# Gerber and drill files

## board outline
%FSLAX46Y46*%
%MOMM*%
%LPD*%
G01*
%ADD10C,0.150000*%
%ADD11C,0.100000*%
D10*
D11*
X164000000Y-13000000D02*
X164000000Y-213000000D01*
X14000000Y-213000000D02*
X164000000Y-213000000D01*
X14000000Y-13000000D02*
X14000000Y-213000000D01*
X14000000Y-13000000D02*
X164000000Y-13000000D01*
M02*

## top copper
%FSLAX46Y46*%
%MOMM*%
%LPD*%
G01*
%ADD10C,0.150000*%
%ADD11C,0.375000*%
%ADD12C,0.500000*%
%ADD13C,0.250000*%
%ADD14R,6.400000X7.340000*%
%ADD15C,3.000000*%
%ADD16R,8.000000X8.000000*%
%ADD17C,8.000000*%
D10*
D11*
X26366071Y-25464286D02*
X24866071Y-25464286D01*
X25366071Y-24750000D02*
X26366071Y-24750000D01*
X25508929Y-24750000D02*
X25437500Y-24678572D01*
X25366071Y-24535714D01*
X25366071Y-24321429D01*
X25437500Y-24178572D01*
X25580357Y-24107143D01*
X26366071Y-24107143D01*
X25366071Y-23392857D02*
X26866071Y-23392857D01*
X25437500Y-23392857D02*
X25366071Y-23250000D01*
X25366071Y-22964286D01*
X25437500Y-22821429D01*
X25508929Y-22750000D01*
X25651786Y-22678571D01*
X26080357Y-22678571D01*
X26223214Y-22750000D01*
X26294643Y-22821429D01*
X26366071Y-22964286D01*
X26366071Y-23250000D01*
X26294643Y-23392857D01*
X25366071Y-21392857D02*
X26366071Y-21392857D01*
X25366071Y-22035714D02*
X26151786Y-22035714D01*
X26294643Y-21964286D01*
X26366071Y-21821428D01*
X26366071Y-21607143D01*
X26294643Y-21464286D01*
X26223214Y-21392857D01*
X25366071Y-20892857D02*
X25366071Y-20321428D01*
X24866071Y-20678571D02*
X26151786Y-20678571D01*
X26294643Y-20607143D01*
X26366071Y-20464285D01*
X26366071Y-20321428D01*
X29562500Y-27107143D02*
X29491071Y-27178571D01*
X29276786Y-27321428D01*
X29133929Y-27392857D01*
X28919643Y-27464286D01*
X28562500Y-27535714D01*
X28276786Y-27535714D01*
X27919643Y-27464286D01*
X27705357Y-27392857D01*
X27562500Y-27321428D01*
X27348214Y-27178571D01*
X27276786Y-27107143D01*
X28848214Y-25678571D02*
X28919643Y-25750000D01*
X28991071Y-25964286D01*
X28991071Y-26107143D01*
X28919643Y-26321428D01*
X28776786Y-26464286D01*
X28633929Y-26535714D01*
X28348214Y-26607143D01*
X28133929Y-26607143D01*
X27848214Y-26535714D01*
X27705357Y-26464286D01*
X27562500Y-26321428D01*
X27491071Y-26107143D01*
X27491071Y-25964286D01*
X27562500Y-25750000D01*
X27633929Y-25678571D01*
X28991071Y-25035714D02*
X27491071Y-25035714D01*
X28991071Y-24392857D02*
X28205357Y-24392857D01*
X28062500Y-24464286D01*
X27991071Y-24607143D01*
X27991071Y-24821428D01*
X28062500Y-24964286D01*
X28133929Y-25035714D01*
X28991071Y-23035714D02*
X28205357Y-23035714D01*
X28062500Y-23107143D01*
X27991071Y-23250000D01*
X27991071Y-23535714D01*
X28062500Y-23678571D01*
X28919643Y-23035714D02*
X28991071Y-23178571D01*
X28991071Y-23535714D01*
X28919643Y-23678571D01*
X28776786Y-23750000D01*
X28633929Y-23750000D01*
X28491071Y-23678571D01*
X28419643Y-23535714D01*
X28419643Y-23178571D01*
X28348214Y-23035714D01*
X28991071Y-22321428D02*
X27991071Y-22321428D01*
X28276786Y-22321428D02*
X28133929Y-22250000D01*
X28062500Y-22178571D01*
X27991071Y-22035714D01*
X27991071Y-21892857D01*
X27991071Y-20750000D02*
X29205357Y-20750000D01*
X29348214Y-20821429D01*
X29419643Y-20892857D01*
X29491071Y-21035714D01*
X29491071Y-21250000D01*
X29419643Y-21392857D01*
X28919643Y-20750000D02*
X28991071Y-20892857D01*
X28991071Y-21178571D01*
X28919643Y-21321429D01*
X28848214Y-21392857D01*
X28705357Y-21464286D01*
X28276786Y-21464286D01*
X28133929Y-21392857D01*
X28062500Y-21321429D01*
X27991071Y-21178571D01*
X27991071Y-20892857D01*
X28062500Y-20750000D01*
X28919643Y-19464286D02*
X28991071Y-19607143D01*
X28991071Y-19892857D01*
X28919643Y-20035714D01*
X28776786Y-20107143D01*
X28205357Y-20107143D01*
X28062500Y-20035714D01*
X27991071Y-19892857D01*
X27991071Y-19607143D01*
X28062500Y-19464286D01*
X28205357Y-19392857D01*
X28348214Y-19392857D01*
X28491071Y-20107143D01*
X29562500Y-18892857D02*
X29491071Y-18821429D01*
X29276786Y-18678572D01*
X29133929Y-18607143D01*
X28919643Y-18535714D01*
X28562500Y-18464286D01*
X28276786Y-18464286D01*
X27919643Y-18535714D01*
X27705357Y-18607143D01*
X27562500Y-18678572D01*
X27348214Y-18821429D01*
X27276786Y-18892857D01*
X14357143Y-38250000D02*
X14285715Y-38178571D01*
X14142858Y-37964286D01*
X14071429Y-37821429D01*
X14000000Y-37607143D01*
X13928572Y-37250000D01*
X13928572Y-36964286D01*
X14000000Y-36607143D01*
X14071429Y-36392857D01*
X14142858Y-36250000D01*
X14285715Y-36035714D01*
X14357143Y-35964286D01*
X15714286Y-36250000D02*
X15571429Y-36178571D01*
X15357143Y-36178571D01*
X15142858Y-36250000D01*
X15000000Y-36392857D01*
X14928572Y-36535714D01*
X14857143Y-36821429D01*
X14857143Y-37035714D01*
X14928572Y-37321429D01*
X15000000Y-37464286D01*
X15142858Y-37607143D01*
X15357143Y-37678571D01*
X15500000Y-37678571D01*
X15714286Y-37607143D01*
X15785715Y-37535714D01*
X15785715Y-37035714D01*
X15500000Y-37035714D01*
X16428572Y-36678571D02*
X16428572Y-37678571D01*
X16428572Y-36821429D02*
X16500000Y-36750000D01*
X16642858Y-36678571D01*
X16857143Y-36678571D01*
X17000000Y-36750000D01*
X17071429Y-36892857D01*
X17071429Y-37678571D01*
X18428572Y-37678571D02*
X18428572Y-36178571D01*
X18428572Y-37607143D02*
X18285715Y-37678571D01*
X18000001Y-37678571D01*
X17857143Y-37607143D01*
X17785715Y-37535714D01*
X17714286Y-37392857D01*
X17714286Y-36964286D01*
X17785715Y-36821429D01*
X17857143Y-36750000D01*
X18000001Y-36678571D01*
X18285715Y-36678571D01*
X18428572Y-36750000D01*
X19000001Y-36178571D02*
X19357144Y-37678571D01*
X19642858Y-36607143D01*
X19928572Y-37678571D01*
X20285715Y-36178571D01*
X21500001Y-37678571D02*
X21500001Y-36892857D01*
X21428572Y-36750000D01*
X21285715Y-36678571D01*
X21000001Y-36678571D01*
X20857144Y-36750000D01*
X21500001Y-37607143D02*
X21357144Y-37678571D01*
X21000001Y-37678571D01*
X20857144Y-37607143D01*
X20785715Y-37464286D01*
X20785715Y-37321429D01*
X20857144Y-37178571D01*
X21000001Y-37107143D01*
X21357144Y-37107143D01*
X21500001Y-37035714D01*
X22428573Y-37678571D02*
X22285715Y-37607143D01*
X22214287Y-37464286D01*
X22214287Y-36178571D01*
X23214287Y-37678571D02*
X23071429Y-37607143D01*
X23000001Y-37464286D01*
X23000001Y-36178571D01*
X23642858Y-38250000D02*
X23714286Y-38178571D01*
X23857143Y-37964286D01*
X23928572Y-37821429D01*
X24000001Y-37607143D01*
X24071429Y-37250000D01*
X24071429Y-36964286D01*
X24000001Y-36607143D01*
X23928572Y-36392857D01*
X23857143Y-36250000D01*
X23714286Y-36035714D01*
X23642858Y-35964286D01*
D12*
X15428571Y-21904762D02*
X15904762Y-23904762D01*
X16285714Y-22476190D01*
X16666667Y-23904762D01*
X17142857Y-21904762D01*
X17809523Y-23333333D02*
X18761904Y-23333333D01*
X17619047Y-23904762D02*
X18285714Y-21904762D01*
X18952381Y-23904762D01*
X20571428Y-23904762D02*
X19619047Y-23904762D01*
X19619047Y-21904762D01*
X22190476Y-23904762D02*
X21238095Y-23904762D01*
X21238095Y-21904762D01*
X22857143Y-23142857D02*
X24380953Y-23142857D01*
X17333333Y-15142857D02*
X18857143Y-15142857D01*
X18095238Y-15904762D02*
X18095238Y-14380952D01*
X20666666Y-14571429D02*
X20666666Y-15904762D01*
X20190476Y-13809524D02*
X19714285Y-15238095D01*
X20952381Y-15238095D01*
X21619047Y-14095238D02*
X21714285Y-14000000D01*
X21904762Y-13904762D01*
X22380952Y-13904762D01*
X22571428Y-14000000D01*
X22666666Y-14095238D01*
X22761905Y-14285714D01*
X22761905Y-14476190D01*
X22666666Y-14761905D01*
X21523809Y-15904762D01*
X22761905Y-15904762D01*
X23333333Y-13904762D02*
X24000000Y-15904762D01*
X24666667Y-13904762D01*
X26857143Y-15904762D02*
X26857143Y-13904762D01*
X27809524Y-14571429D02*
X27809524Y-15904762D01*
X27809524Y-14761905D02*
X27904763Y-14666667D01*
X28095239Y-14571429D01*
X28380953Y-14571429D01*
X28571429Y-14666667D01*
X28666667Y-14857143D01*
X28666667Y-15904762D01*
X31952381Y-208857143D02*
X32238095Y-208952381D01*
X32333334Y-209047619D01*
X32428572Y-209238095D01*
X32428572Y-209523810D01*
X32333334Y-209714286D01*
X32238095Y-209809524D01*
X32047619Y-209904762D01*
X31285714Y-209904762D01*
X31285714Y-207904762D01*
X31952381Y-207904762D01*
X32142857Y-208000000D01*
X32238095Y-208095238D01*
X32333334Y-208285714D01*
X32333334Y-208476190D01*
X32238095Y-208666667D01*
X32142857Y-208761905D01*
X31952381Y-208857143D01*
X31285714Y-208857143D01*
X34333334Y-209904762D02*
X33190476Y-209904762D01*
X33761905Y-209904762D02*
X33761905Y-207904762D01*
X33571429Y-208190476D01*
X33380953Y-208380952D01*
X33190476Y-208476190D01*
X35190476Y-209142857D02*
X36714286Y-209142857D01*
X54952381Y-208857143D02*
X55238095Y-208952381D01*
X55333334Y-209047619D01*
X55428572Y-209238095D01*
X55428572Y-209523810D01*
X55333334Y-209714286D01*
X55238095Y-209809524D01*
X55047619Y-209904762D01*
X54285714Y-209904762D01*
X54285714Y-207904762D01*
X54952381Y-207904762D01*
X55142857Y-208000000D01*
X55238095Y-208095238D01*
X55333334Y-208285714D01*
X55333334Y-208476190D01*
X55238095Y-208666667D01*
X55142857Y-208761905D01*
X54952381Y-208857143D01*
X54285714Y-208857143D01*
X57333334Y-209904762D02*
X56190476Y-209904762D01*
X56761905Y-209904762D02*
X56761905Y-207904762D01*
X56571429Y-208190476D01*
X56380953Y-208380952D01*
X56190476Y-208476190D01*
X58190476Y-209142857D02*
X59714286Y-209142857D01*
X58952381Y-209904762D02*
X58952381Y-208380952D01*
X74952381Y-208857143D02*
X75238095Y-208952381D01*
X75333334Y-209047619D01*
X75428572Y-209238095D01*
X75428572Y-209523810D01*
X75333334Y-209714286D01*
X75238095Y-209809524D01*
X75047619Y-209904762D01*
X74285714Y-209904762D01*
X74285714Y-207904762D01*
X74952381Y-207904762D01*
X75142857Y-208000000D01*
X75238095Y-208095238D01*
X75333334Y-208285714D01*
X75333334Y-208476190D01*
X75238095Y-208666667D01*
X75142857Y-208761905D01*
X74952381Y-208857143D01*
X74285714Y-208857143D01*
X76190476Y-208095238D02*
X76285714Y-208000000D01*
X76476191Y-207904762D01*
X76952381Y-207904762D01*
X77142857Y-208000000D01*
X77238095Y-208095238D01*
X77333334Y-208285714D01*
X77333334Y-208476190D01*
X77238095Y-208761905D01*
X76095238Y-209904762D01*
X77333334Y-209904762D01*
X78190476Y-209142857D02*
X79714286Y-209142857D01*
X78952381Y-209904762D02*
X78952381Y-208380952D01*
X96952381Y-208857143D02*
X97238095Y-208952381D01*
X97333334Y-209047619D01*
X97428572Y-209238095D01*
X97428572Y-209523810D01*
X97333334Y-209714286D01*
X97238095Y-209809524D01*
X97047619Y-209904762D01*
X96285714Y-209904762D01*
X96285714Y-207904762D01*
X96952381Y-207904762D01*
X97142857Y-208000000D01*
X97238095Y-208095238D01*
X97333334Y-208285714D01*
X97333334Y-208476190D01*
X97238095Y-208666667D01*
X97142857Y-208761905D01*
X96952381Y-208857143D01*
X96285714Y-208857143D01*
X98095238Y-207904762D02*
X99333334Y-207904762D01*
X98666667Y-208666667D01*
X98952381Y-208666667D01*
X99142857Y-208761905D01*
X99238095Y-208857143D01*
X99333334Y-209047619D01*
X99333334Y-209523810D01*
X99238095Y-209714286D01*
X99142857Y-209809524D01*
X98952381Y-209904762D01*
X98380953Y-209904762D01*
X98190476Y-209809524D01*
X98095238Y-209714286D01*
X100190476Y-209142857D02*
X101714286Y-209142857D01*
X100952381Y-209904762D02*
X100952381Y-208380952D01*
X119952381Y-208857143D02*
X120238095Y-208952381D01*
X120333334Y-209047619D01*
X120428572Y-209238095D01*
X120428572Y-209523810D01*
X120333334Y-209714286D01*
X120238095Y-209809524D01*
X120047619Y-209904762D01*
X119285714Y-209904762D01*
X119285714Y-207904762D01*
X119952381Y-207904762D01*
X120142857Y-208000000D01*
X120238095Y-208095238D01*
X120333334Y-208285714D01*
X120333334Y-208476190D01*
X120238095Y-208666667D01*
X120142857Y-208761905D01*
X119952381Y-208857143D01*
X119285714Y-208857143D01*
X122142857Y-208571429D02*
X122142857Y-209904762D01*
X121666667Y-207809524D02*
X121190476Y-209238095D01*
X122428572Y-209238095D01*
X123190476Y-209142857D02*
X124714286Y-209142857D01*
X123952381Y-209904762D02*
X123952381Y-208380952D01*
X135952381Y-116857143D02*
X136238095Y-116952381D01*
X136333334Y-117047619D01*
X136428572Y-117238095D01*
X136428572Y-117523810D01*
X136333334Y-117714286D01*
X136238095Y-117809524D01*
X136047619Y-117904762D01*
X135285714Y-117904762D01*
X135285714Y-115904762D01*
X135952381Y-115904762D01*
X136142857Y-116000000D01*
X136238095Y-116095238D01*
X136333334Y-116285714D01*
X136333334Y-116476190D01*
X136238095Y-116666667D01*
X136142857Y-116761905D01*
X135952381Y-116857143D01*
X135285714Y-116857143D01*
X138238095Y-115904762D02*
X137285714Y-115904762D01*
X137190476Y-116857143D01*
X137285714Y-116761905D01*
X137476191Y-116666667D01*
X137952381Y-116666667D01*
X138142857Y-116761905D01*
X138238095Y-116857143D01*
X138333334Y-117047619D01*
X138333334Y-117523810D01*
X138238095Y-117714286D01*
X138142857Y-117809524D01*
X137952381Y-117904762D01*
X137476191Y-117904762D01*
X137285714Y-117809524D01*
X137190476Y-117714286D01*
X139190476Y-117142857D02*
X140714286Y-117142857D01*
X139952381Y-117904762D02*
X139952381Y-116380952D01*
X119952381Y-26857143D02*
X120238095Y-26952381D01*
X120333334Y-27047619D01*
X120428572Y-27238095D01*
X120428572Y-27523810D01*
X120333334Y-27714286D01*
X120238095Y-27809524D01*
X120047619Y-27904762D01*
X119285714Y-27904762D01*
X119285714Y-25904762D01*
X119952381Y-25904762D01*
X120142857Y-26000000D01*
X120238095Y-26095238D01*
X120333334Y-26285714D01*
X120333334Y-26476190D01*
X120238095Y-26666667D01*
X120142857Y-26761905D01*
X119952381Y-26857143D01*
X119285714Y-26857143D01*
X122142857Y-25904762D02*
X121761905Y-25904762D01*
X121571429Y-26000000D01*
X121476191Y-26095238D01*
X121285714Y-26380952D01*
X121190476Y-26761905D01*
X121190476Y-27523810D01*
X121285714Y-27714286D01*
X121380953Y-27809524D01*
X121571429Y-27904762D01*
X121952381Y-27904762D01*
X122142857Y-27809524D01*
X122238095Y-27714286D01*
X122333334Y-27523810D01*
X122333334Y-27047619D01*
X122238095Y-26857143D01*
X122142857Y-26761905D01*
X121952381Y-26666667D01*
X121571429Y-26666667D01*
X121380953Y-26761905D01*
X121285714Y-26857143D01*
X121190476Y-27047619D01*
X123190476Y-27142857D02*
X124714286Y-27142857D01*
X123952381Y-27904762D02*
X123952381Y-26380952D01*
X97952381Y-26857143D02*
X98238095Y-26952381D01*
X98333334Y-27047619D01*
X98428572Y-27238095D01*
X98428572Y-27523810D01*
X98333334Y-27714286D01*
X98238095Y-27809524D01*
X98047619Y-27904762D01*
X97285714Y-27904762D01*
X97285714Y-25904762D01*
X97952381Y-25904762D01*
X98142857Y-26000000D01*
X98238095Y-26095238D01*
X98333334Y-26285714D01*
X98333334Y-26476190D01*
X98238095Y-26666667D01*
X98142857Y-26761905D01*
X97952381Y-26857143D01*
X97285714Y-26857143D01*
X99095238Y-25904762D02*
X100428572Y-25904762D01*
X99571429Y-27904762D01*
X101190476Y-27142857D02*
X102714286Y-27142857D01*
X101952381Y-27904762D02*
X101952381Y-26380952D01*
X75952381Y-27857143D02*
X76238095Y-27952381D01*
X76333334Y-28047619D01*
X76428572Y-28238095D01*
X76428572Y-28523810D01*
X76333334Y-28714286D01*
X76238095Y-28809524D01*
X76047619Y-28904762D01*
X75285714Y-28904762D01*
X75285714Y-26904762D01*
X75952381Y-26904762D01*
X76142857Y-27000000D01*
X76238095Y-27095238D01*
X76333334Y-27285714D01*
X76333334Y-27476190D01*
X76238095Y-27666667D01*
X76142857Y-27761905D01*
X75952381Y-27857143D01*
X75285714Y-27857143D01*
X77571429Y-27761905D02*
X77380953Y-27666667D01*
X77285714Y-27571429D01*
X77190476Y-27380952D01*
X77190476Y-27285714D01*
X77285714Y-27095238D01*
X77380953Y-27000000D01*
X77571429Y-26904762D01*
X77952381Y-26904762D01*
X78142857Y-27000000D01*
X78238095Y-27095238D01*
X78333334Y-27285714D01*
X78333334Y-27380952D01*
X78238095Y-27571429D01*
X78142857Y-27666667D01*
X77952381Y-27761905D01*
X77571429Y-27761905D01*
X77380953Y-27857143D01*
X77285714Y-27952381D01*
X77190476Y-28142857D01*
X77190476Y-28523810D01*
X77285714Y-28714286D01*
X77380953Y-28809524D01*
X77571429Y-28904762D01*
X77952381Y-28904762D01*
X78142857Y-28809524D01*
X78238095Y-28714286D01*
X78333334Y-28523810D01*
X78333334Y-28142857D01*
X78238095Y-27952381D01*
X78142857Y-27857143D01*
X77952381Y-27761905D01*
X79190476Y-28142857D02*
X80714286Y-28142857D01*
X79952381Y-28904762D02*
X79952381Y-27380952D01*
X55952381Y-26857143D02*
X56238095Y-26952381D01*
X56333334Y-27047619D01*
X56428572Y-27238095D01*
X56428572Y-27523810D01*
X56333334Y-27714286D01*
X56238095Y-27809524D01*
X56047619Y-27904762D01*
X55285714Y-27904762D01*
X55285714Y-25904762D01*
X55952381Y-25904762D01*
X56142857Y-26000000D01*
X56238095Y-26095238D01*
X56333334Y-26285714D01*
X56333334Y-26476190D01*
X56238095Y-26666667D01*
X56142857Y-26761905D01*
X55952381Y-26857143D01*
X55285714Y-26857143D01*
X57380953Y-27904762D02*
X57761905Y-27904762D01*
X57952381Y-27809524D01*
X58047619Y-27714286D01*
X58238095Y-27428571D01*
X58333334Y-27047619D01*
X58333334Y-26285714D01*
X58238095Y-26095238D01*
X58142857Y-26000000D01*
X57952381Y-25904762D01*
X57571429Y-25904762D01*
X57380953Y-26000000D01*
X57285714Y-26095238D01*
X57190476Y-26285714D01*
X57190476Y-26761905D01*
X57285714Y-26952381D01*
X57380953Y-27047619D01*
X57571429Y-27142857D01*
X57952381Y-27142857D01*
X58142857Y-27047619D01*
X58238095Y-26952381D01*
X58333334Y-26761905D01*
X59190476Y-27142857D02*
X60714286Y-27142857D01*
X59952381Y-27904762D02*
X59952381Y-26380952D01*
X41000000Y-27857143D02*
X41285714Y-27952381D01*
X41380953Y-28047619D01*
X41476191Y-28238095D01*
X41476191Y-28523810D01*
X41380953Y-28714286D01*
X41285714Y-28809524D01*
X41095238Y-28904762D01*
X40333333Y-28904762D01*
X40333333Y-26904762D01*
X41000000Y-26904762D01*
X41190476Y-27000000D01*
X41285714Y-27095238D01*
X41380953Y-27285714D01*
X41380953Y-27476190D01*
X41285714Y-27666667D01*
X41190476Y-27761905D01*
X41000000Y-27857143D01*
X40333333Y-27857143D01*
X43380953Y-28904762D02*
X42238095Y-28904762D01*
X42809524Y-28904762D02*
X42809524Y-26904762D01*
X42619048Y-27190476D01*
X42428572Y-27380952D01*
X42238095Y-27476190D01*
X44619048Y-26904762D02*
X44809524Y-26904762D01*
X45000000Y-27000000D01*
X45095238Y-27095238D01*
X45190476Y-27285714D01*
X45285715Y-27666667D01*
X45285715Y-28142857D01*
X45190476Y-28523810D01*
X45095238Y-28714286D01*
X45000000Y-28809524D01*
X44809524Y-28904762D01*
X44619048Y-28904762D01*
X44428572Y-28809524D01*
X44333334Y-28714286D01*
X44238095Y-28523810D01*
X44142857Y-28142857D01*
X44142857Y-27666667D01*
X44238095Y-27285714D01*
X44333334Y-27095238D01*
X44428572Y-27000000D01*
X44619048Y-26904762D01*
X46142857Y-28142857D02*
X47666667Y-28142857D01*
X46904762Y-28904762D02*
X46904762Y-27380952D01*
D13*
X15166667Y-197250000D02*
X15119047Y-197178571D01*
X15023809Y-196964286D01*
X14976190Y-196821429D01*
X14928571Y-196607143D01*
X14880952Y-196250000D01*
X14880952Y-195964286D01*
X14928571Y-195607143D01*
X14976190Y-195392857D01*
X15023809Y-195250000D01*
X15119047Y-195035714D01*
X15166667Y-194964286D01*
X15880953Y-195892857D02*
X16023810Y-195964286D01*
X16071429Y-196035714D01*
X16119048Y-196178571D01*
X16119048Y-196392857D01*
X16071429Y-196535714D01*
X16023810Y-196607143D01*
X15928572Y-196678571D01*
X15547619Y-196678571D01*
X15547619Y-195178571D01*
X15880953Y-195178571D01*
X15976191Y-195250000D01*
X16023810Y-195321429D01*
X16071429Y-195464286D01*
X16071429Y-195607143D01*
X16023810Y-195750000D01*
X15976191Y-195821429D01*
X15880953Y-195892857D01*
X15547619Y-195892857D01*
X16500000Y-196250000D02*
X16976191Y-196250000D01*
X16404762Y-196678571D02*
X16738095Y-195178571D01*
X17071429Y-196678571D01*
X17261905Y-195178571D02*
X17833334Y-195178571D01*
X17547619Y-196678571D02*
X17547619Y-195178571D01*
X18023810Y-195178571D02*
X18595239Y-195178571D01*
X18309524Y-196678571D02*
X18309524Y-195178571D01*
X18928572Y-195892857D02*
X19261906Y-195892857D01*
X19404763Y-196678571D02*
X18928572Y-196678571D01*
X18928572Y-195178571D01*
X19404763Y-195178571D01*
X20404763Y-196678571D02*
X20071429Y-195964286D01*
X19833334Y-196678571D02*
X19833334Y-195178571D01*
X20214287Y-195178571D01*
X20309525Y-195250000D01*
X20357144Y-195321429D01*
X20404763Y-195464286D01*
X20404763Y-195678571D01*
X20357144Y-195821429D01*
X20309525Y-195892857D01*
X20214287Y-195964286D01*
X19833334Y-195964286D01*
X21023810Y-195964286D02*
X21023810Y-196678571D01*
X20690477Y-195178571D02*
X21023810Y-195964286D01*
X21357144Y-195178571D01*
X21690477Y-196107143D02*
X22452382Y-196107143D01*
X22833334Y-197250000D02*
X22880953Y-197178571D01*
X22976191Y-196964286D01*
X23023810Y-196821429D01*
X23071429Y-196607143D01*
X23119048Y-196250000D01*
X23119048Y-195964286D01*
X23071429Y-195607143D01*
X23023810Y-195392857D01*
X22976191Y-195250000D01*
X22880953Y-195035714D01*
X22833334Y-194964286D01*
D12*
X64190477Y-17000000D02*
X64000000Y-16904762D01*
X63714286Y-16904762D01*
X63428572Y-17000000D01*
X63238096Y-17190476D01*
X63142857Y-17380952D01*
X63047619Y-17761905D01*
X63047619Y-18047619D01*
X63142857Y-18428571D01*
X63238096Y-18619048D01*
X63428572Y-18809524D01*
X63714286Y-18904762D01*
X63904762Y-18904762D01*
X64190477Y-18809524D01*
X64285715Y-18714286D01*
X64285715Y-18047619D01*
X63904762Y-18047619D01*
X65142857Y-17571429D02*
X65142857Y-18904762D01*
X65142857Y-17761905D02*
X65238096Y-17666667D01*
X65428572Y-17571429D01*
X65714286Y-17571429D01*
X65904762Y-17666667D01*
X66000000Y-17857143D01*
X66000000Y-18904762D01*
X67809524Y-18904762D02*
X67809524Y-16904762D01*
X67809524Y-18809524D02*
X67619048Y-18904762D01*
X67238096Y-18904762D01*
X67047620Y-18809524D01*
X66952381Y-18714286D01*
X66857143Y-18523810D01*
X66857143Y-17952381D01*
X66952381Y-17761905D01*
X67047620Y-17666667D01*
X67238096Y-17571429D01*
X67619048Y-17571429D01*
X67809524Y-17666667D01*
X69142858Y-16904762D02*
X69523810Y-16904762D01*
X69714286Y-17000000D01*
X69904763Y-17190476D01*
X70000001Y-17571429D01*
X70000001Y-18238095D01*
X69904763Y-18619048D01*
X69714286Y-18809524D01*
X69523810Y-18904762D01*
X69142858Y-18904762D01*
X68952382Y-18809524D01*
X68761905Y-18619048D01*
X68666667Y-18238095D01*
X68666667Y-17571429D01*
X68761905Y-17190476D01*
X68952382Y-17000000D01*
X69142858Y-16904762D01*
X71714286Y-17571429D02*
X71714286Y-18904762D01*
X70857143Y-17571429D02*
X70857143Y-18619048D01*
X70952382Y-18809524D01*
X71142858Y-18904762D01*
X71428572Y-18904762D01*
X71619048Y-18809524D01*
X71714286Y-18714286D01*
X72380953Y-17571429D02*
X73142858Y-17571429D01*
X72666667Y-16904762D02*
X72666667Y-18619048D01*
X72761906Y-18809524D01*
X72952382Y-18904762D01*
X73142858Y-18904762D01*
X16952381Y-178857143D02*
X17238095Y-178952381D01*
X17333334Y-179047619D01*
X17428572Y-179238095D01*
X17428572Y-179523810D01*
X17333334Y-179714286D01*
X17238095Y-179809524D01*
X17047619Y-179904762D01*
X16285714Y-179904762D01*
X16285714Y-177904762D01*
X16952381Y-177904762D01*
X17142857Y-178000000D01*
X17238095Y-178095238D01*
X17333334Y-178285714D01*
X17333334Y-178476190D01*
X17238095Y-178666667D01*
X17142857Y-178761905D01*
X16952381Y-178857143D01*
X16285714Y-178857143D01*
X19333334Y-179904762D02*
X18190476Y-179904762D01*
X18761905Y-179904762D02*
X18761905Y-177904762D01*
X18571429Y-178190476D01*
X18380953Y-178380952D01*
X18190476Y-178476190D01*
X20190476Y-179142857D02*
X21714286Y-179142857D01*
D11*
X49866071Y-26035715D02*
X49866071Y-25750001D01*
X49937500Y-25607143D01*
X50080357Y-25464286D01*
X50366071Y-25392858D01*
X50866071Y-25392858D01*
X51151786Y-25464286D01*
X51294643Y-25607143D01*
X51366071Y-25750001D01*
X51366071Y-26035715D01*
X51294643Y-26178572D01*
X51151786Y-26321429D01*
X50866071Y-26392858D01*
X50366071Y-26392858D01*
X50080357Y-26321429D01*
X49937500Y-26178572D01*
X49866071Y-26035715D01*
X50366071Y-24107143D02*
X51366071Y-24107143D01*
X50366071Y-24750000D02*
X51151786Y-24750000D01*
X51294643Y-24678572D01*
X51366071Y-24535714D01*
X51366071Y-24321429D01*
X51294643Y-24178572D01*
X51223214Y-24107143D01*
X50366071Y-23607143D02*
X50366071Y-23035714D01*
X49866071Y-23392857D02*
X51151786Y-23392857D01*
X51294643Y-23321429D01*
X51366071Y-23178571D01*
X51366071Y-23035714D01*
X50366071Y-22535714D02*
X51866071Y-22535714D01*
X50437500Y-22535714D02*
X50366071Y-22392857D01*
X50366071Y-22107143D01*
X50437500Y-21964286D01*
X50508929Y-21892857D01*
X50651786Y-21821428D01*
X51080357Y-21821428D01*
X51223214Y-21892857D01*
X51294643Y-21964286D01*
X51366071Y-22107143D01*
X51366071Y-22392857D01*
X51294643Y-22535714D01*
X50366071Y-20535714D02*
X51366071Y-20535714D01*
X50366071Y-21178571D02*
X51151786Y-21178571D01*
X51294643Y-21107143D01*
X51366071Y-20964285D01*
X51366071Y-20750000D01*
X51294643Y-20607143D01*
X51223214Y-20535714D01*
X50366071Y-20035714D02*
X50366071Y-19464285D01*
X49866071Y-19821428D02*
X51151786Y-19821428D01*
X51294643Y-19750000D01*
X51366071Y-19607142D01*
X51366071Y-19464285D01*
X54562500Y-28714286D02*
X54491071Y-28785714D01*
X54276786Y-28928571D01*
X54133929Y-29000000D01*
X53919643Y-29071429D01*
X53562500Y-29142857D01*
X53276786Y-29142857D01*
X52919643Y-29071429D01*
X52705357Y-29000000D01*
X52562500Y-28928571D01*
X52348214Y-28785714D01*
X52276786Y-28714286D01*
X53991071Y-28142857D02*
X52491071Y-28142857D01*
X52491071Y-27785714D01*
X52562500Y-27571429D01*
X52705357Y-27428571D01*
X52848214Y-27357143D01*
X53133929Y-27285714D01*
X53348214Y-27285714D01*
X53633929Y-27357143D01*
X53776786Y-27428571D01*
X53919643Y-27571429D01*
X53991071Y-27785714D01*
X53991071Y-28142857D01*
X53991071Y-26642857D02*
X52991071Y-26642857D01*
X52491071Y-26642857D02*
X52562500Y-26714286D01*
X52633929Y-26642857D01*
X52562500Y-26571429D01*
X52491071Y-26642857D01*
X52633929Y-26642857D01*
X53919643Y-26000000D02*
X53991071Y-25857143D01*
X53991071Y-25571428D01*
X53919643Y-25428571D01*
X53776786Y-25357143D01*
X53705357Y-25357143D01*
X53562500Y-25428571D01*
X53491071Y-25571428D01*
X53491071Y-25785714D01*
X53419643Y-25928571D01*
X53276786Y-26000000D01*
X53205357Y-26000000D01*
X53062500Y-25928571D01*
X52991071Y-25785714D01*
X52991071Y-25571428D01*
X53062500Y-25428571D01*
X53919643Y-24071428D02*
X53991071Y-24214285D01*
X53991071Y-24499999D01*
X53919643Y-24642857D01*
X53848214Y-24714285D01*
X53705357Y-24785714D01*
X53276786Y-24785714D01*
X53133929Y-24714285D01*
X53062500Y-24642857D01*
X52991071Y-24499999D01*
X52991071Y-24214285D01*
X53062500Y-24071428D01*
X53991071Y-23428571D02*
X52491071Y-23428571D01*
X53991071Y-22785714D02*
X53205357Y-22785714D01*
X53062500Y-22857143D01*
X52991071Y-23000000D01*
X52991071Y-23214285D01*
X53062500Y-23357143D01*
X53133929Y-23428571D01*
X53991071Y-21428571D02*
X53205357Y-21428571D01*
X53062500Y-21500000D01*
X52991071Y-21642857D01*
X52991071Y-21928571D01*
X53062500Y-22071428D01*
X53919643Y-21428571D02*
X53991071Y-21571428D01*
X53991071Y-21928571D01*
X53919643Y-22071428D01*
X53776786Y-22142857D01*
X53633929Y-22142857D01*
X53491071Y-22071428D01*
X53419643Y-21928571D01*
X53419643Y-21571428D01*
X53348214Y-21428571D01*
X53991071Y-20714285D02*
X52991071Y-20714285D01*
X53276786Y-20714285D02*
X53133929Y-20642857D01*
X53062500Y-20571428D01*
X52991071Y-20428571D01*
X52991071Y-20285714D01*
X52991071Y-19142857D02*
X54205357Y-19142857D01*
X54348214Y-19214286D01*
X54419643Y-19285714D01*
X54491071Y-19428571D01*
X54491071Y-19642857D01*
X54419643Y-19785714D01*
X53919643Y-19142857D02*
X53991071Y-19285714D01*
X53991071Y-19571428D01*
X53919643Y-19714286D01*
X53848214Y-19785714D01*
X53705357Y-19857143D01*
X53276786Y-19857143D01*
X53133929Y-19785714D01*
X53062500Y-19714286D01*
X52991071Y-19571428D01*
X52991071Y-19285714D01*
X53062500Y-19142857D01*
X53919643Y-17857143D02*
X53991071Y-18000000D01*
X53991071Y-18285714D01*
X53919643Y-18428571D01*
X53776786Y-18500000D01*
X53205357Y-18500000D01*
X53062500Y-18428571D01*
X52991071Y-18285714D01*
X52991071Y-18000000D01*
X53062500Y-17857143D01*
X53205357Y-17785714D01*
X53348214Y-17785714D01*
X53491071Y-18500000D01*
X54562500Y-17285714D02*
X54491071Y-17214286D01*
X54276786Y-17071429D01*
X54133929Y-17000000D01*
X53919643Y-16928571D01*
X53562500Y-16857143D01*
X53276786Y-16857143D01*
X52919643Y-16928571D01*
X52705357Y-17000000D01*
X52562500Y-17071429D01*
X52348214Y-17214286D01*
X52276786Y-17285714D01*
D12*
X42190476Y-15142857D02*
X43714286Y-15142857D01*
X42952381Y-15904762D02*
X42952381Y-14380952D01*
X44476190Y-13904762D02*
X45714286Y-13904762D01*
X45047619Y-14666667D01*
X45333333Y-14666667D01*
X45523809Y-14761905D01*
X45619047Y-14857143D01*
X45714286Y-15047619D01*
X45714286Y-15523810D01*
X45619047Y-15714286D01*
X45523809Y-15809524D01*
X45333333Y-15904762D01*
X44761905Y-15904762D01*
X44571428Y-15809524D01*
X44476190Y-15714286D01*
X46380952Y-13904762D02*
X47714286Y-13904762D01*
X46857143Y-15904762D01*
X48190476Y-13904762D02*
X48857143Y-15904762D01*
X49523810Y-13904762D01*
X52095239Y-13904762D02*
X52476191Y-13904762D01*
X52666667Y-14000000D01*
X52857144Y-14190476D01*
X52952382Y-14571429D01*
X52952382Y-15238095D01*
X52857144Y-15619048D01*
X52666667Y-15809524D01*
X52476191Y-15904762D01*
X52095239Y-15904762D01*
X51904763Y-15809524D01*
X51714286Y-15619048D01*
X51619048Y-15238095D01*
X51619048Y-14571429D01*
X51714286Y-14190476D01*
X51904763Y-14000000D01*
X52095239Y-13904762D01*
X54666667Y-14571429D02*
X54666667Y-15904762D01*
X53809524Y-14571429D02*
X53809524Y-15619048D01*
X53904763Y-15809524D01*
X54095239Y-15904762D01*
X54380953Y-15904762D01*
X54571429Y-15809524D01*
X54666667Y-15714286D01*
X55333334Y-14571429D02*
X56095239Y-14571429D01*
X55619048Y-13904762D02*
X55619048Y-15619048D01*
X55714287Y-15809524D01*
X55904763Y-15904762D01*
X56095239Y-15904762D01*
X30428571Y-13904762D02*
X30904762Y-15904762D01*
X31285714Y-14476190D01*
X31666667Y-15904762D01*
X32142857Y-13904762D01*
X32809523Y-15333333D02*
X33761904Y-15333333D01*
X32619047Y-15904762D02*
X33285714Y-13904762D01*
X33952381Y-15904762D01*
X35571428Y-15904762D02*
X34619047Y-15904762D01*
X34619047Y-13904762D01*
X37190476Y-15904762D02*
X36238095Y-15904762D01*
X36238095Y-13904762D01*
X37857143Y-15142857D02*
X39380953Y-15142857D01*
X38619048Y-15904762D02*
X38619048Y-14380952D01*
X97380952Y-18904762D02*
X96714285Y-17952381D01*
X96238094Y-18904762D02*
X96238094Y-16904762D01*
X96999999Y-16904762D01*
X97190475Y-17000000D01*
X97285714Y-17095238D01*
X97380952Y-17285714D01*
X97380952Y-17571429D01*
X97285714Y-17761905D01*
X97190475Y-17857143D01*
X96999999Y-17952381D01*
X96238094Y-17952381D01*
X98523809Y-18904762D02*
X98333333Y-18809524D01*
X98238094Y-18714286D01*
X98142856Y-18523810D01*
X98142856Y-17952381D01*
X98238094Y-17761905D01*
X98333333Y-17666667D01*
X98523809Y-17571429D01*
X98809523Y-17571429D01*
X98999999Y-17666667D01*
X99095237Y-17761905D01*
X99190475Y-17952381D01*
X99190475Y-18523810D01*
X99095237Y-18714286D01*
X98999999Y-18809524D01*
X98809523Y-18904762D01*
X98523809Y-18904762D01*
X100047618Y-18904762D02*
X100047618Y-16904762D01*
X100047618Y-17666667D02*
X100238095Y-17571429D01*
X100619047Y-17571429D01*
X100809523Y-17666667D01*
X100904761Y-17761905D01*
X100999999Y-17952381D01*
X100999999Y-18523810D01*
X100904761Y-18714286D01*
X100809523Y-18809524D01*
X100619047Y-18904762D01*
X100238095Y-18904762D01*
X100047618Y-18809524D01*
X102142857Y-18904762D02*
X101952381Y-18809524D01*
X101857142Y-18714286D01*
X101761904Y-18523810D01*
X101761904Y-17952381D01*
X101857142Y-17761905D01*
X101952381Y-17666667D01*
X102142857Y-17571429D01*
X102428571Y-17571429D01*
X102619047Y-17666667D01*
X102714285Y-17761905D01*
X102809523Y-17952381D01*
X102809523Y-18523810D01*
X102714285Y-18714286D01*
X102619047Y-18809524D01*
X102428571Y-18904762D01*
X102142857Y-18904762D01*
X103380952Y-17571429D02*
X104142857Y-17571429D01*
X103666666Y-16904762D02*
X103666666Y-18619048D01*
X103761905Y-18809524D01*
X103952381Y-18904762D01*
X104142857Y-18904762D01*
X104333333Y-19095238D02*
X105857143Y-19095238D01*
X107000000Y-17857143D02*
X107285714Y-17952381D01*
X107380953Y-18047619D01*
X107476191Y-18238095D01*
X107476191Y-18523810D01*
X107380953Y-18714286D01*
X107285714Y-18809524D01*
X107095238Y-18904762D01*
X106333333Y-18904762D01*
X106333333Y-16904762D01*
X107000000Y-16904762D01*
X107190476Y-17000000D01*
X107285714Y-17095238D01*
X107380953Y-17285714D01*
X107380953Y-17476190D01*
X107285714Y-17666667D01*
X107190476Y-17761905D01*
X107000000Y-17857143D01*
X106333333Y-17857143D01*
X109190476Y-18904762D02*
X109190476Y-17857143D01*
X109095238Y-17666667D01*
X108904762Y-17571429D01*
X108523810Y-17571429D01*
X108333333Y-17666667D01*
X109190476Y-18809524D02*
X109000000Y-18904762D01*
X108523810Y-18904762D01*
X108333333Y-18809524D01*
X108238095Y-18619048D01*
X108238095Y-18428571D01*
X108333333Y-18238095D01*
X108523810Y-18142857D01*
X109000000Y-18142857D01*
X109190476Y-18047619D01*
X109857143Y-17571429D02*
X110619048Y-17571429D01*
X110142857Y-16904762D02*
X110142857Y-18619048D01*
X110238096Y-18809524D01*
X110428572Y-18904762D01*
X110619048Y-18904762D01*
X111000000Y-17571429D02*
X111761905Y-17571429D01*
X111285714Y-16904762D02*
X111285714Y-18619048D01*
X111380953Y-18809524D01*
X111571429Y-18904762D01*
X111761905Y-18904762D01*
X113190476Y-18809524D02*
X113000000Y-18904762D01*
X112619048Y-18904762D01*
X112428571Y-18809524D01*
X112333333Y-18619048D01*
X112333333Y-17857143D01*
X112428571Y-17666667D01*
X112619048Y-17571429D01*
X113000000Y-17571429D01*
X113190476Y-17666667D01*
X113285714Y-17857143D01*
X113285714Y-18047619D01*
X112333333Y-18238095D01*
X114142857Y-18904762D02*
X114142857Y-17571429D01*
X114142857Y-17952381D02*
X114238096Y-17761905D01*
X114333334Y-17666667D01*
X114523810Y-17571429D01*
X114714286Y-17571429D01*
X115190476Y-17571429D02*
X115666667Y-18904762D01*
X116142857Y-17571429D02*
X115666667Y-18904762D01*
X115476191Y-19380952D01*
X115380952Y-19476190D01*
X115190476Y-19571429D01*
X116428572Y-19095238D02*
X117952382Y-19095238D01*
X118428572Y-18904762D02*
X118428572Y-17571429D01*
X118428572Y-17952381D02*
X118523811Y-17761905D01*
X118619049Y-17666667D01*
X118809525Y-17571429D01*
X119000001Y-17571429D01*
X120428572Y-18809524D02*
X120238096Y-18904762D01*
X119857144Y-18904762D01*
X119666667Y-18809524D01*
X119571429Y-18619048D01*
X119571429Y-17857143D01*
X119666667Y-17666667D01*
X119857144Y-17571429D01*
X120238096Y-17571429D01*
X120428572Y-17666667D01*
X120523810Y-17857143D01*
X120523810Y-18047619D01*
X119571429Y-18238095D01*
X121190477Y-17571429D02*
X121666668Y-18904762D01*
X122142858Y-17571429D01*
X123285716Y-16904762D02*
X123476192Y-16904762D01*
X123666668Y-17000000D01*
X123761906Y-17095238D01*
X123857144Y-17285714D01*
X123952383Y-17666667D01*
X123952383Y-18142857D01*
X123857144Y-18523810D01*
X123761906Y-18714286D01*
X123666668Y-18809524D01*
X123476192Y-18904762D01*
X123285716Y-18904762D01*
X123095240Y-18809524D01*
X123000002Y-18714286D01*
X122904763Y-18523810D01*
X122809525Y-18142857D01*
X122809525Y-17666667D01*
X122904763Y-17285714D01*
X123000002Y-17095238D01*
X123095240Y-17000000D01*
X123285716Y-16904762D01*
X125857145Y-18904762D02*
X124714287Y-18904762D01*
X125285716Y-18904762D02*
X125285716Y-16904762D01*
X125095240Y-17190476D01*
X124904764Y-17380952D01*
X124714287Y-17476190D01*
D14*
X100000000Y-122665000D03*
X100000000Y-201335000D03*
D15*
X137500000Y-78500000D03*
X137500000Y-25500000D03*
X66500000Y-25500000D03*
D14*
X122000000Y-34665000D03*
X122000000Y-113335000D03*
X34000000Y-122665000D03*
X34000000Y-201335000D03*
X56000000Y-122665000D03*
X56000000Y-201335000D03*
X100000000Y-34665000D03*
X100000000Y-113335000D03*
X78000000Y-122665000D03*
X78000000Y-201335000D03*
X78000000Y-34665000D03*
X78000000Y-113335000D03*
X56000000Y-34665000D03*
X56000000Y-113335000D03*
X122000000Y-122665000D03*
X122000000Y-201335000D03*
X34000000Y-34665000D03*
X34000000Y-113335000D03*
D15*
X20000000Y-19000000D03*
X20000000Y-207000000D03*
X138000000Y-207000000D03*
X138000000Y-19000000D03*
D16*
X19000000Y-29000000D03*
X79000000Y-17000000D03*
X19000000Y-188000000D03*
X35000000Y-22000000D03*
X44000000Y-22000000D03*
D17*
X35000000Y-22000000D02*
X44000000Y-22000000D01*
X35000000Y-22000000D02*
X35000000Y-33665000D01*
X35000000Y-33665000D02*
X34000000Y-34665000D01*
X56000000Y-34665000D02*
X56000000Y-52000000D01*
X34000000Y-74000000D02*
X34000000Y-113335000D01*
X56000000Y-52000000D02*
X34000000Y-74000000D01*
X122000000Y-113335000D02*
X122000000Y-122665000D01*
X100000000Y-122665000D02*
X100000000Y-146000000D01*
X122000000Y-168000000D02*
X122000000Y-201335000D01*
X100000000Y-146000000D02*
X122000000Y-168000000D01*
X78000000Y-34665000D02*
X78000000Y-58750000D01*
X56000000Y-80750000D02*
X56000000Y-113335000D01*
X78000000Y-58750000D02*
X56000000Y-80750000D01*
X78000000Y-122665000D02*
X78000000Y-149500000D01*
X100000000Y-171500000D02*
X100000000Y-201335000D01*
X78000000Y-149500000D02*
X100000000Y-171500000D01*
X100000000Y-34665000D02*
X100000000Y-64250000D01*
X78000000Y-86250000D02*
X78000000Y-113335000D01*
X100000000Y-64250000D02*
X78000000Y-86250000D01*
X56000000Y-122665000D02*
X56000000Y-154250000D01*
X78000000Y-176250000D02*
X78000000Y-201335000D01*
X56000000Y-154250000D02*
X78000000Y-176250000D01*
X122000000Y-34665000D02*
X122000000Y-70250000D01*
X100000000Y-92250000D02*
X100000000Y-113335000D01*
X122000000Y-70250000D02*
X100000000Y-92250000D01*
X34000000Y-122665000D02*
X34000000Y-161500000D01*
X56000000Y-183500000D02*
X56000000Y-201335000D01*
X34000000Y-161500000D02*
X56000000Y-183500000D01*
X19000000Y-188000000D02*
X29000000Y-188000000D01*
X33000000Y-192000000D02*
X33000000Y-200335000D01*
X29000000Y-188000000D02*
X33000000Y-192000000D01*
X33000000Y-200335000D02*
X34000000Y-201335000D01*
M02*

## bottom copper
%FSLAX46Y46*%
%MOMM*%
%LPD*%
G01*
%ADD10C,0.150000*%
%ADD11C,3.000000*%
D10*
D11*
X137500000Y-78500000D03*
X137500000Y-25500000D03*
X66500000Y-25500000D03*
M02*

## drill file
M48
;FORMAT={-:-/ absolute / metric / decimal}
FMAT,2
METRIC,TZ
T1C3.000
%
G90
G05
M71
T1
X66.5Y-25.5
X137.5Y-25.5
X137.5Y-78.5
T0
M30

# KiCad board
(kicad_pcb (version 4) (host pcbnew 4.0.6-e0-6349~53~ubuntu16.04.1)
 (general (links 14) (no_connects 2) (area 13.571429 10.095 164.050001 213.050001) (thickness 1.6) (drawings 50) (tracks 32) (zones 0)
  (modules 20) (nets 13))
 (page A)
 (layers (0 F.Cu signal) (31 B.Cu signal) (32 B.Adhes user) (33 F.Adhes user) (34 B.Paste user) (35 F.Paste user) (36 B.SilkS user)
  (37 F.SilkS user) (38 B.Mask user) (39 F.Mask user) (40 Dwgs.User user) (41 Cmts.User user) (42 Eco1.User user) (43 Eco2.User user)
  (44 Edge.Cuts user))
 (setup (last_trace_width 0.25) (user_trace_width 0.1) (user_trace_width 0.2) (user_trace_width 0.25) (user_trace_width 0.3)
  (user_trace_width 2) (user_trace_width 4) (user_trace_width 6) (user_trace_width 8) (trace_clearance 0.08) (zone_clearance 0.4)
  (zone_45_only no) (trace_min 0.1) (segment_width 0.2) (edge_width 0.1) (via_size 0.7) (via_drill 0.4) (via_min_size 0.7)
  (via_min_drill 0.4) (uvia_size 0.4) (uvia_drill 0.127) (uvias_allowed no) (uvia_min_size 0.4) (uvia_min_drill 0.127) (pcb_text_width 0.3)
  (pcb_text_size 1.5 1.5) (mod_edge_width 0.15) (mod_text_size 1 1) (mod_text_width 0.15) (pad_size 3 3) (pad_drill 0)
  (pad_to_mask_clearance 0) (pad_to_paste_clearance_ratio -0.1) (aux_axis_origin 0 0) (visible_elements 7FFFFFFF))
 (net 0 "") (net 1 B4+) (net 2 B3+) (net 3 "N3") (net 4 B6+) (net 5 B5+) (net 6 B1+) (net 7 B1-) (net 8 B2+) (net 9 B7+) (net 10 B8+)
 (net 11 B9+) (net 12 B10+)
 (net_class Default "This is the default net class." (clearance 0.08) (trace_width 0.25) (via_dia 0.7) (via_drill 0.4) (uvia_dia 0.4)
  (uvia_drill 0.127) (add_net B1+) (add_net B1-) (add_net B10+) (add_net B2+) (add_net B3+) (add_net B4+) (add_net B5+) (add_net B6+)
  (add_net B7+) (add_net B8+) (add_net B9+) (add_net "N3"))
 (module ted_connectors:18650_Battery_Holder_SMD (layer F.Cu) (at 100 162 270)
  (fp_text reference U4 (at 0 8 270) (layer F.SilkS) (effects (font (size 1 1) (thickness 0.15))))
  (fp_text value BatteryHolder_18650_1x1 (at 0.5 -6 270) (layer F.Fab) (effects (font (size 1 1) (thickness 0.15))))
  (pad 1 smd rect (at -39.335 0 270) (size 7.34 6.4) (layers F.Cu F.Paste F.Mask) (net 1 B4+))
  (pad 2 smd rect (at 39.335 0 270) (size 7.34 6.4) (layers F.Cu F.Paste F.Mask) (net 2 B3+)))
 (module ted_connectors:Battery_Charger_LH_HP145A (layer F.Cu) (at 102 52 90)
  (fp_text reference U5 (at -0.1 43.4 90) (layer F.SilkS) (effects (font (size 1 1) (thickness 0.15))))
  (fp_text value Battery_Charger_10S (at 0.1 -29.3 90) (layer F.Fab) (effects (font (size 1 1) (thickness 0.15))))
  (pad 1 thru_hole circle (at -26.5 35.5 90) (size 3 3) (drill 3) (layers *.Cu *.Mask) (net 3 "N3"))
  (pad 1 thru_hole circle (at 26.5 35.5 90) (size 3 3) (drill 3) (layers *.Cu *.Mask) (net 3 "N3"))
  (pad 1 thru_hole circle (at 26.5 -35.5 90) (size 3 3) (drill 3) (layers *.Cu *.Mask) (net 3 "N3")))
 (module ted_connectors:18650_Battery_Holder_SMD (layer F.Cu) (at 122 74 270)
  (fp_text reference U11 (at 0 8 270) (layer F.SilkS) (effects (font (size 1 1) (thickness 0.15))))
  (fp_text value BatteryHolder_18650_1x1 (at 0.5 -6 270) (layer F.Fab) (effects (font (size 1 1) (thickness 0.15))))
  (pad 1 smd rect (at -39.335 0 270) (size 7.34 6.4) (layers F.Cu F.Paste F.Mask) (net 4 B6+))
  (pad 2 smd rect (at 39.335 0 270) (size 7.34 6.4) (layers F.Cu F.Paste F.Mask) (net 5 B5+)))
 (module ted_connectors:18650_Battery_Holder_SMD (layer F.Cu) (at 34 162 270)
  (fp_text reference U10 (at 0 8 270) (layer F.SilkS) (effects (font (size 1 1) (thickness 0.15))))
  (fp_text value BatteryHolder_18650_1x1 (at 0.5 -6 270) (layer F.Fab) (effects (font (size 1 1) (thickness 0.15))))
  (pad 1 smd rect (at -39.335 0 270) (size 7.34 6.4) (layers F.Cu F.Paste F.Mask) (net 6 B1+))
  (pad 2 smd rect (at 39.335 0 270) (size 7.34 6.4) (layers F.Cu F.Paste F.Mask) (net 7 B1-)))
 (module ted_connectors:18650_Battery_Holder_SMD (layer F.Cu) (at 56 162 270)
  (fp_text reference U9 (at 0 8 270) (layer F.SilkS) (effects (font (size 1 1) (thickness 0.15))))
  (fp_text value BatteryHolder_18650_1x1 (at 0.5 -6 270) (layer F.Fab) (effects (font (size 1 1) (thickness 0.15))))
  (pad 1 smd rect (at -39.335 0 270) (size 7.34 6.4) (layers F.Cu F.Paste F.Mask) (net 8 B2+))
  (pad 2 smd rect (at 39.335 0 270) (size 7.34 6.4) (layers F.Cu F.Paste F.Mask) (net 6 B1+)))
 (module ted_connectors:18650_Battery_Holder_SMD (layer F.Cu) (at 100 74 270)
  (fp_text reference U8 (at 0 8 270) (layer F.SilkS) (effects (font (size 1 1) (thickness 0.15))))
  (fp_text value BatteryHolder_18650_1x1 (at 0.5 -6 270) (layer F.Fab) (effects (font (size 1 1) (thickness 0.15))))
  (pad 1 smd rect (at -39.335 0 270) (size 7.34 6.4) (layers F.Cu F.Paste F.Mask) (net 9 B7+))
  (pad 2 smd rect (at 39.335 0 270) (size 7.34 6.4) (layers F.Cu F.Paste F.Mask) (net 4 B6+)))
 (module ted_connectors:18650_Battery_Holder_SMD (layer F.Cu) (at 78 162 270)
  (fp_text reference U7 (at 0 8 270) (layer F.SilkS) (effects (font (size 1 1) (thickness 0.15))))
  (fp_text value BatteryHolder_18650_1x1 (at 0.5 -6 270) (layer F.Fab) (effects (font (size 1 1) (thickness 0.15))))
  (pad 1 smd rect (at -39.335 0 270) (size 7.34 6.4) (layers F.Cu F.Paste F.Mask) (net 2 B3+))
  (pad 2 smd rect (at 39.335 0 270) (size 7.34 6.4) (layers F.Cu F.Paste F.Mask) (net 8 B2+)))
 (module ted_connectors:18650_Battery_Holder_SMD (layer F.Cu) (at 78 74 270)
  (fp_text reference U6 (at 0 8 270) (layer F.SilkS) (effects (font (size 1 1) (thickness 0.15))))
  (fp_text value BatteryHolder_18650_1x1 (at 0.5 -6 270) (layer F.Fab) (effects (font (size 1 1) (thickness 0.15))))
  (pad 1 smd rect (at -39.335 0 270) (size 7.34 6.4) (layers F.Cu F.Paste F.Mask) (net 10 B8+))
  (pad 2 smd rect (at 39.335 0 270) (size 7.34 6.4) (layers F.Cu F.Paste F.Mask) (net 9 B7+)))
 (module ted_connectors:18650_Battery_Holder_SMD (layer F.Cu) (at 56 74 270)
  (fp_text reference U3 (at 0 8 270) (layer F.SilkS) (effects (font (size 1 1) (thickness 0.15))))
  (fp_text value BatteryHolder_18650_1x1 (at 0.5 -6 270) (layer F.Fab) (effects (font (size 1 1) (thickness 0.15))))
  (pad 1 smd rect (at -39.335 0 270) (size 7.34 6.4) (layers F.Cu F.Paste F.Mask) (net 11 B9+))
  (pad 2 smd rect (at 39.335 0 270) (size 7.34 6.4) (layers F.Cu F.Paste F.Mask) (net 10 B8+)))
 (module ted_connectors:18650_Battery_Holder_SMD (layer F.Cu) (at 122 162 270)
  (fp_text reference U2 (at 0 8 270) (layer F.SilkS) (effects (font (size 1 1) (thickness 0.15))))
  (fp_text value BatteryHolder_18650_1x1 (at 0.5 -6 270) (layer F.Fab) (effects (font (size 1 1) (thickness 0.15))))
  (pad 1 smd rect (at -39.335 0 270) (size 7.34 6.4) (layers F.Cu F.Paste F.Mask) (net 5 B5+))
  (pad 2 smd rect (at 39.335 0 270) (size 7.34 6.4) (layers F.Cu F.Paste F.Mask) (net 1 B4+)))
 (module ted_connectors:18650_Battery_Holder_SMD (layer F.Cu) (at 34 74 270)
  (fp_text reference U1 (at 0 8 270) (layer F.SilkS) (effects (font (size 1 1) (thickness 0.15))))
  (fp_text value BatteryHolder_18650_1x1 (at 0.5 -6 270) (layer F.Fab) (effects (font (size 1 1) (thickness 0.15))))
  (pad 1 smd rect (at -39.335 0 270) (size 7.34 6.4) (layers F.Cu F.Paste F.Mask) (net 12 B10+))
  (pad 2 smd rect (at 39.335 0 270) (size 7.34 6.4) (layers F.Cu F.Paste F.Mask) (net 11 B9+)))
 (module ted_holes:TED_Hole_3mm (layer F.Cu) (at 20 19)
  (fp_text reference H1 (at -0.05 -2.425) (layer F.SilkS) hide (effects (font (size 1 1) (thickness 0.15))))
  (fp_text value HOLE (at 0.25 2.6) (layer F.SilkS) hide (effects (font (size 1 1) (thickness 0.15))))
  (pad "" connect circle (at 0 0) (size 3 3) (layers F.Cu F.Mask)))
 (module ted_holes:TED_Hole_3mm (layer F.Cu) (at 20 207)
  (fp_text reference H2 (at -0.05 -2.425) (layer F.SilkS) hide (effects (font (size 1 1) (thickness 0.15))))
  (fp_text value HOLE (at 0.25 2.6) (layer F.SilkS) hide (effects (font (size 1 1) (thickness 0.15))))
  (pad "" connect circle (at 0 0) (size 3 3) (layers F.Cu F.Mask)))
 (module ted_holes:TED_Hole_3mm (layer F.Cu) (at 138 207)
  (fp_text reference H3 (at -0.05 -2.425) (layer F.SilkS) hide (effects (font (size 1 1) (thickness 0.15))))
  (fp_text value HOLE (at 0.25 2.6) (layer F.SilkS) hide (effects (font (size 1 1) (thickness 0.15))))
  (pad "" connect circle (at 0 0) (size 3 3) (layers F.Cu F.Mask)))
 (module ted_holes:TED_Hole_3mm (layer F.Cu) (at 138 19)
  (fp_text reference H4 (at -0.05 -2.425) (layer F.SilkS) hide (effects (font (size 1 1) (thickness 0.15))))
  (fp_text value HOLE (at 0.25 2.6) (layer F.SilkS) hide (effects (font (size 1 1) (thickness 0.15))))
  (pad "" connect circle (at 0 0) (size 3 3) (layers F.Cu F.Mask)))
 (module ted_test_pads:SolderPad (layer F.Cu) (at 19 29)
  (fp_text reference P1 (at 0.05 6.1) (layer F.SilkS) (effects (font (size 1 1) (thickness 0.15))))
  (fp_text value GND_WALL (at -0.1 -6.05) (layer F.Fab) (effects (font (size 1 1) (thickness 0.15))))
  (pad 1 smd rect (at 0 0) (size 8 8) (layers F.Cu F.Paste F.Mask)))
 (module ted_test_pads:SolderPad (layer F.Cu) (at 79 17)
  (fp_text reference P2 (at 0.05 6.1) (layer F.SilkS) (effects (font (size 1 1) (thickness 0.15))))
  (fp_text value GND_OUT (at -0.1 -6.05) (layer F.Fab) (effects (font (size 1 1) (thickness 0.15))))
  (pad 1 smd rect (at 0 0) (size 8 8) (layers F.Cu F.Paste F.Mask)))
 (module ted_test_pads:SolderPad (layer F.Cu) (at 19 188)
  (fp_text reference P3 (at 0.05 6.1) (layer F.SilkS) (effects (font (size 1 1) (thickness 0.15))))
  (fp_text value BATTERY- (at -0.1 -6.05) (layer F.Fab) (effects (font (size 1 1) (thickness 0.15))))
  (pad 1 smd rect (at 0 0) (size 8 8) (layers F.Cu F.Paste F.Mask) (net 7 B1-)))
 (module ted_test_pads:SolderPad (layer F.Cu) (at 35 22)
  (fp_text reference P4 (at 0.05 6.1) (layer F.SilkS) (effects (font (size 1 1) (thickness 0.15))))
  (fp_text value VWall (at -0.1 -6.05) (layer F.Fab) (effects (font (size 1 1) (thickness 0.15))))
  (pad 1 smd rect (at 0 0) (size 8 8) (layers F.Cu F.Paste F.Mask) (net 12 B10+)))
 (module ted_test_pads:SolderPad (layer F.Cu) (at 44 22)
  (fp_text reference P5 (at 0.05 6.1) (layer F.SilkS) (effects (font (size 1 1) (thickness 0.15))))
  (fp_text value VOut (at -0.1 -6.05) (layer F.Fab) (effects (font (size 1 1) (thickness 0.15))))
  (pad 1 smd rect (at 0 0) (size 8 8) (layers F.Cu F.Paste F.Mask) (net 12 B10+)))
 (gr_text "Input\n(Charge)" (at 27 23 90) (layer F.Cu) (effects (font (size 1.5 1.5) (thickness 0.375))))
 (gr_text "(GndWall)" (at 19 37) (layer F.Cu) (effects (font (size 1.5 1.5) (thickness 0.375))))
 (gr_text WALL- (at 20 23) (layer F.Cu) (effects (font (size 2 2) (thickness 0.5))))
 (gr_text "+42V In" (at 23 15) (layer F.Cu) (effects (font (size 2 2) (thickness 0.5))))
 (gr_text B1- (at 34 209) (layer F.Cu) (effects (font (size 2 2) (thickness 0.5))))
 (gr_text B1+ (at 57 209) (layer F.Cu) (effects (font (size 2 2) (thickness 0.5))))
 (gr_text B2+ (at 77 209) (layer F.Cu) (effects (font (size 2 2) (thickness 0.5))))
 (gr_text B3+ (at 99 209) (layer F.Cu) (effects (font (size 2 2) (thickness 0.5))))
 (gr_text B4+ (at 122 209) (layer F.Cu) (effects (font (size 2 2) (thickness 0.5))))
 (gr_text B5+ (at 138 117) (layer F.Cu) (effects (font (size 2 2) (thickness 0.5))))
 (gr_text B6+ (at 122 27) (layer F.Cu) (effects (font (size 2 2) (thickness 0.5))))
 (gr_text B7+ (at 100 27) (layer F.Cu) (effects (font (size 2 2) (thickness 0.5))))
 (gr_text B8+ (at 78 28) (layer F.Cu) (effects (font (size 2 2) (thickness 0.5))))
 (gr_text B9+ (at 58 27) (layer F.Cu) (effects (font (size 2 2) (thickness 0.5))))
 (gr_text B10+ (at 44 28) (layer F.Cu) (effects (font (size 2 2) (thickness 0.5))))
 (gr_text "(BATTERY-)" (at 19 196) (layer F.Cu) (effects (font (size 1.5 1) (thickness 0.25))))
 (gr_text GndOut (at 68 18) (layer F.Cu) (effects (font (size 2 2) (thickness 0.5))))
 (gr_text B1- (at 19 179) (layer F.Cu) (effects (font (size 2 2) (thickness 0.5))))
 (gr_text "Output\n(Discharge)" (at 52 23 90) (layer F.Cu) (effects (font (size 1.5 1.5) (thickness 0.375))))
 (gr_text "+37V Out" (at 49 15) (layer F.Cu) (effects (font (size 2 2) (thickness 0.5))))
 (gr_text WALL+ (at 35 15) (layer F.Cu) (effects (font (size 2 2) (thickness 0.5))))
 (gr_line (start 164 13) (end 164 213) (angle 90) (layer Edge.Cuts) (width 0.1))
 (gr_line (start 14 213) (end 164 213) (angle 90) (layer Edge.Cuts) (width 0.1))
 (gr_line (start 14 13) (end 14 213) (angle 90) (layer Edge.Cuts) (width 0.1))
 (gr_line (start 14 13) (end 164 13) (angle 90) (layer Edge.Cuts) (width 0.1))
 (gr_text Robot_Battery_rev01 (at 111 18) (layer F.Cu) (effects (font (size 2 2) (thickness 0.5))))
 (segment (start 35 22) (end 44 22) (width 8) (layer F.Cu) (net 12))
 (segment (start 35 22) (end 35 33.665) (width 8) (layer F.Cu) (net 12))
 (segment (start 35 33.665) (end 34 34.665) (width 8) (layer F.Cu) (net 12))
 (segment (start 56 34.665) (end 56 52) (width 8) (layer F.Cu) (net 11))
 (segment (start 34 74) (end 34 113.335) (width 8) (layer F.Cu) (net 11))
 (segment (start 56 52) (end 34 74) (width 8) (layer F.Cu) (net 11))
 (segment (start 122 113.335) (end 122 122.665) (width 8) (layer F.Cu) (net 5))
 (segment (start 100 122.665) (end 100 146) (width 8) (layer F.Cu) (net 1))
 (segment (start 122 168) (end 122 201.335) (width 8) (layer F.Cu) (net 1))
 (segment (start 100 146) (end 122 168) (width 8) (layer F.Cu) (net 1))
 (segment (start 78 34.665) (end 78 58.75) (width 8) (layer F.Cu) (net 10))
 (segment (start 56 80.75) (end 56 113.335) (width 8) (layer F.Cu) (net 10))
 (segment (start 78 58.75) (end 56 80.75) (width 8) (layer F.Cu) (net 10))
 (segment (start 78 122.665) (end 78 149.5) (width 8) (layer F.Cu) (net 2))
 (segment (start 100 171.5) (end 100 201.335) (width 8) (layer F.Cu) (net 2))
 (segment (start 78 149.5) (end 100 171.5) (width 8) (layer F.Cu) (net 2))
 (segment (start 100 34.665) (end 100 64.25) (width 8) (layer F.Cu) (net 9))
 (segment (start 78 86.25) (end 78 113.335) (width 8) (layer F.Cu) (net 9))
 (segment (start 100 64.25) (end 78 86.25) (width 8) (layer F.Cu) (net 9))
 (segment (start 56 122.665) (end 56 154.25) (width 8) (layer F.Cu) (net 8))
 (segment (start 78 176.25) (end 78 201.335) (width 8) (layer F.Cu) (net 8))
 (segment (start 56 154.25) (end 78 176.25) (width 8) (layer F.Cu) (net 8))
 (segment (start 122 34.665) (end 122 70.25) (width 8) (layer F.Cu) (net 4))
 (segment (start 100 92.25) (end 100 113.335) (width 8) (layer F.Cu) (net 4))
 (segment (start 122 70.25) (end 100 92.25) (width 8) (layer F.Cu) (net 4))
 (segment (start 34 122.665) (end 34 161.5) (width 8) (layer F.Cu) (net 6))
 (segment (start 56 183.5) (end 56 201.335) (width 8) (layer F.Cu) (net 6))
 (segment (start 34 161.5) (end 56 183.5) (width 8) (layer F.Cu) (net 6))
 (segment (start 19 188) (end 29 188) (width 8) (layer F.Cu) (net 7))
 (segment (start 33 192) (end 33 200.335) (width 8) (layer F.Cu) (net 7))
 (segment (start 29 188) (end 33 192) (width 8) (layer F.Cu) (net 7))
 (segment (start 33 200.335) (end 34 201.335) (width 8) (layer F.Cu) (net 7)))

